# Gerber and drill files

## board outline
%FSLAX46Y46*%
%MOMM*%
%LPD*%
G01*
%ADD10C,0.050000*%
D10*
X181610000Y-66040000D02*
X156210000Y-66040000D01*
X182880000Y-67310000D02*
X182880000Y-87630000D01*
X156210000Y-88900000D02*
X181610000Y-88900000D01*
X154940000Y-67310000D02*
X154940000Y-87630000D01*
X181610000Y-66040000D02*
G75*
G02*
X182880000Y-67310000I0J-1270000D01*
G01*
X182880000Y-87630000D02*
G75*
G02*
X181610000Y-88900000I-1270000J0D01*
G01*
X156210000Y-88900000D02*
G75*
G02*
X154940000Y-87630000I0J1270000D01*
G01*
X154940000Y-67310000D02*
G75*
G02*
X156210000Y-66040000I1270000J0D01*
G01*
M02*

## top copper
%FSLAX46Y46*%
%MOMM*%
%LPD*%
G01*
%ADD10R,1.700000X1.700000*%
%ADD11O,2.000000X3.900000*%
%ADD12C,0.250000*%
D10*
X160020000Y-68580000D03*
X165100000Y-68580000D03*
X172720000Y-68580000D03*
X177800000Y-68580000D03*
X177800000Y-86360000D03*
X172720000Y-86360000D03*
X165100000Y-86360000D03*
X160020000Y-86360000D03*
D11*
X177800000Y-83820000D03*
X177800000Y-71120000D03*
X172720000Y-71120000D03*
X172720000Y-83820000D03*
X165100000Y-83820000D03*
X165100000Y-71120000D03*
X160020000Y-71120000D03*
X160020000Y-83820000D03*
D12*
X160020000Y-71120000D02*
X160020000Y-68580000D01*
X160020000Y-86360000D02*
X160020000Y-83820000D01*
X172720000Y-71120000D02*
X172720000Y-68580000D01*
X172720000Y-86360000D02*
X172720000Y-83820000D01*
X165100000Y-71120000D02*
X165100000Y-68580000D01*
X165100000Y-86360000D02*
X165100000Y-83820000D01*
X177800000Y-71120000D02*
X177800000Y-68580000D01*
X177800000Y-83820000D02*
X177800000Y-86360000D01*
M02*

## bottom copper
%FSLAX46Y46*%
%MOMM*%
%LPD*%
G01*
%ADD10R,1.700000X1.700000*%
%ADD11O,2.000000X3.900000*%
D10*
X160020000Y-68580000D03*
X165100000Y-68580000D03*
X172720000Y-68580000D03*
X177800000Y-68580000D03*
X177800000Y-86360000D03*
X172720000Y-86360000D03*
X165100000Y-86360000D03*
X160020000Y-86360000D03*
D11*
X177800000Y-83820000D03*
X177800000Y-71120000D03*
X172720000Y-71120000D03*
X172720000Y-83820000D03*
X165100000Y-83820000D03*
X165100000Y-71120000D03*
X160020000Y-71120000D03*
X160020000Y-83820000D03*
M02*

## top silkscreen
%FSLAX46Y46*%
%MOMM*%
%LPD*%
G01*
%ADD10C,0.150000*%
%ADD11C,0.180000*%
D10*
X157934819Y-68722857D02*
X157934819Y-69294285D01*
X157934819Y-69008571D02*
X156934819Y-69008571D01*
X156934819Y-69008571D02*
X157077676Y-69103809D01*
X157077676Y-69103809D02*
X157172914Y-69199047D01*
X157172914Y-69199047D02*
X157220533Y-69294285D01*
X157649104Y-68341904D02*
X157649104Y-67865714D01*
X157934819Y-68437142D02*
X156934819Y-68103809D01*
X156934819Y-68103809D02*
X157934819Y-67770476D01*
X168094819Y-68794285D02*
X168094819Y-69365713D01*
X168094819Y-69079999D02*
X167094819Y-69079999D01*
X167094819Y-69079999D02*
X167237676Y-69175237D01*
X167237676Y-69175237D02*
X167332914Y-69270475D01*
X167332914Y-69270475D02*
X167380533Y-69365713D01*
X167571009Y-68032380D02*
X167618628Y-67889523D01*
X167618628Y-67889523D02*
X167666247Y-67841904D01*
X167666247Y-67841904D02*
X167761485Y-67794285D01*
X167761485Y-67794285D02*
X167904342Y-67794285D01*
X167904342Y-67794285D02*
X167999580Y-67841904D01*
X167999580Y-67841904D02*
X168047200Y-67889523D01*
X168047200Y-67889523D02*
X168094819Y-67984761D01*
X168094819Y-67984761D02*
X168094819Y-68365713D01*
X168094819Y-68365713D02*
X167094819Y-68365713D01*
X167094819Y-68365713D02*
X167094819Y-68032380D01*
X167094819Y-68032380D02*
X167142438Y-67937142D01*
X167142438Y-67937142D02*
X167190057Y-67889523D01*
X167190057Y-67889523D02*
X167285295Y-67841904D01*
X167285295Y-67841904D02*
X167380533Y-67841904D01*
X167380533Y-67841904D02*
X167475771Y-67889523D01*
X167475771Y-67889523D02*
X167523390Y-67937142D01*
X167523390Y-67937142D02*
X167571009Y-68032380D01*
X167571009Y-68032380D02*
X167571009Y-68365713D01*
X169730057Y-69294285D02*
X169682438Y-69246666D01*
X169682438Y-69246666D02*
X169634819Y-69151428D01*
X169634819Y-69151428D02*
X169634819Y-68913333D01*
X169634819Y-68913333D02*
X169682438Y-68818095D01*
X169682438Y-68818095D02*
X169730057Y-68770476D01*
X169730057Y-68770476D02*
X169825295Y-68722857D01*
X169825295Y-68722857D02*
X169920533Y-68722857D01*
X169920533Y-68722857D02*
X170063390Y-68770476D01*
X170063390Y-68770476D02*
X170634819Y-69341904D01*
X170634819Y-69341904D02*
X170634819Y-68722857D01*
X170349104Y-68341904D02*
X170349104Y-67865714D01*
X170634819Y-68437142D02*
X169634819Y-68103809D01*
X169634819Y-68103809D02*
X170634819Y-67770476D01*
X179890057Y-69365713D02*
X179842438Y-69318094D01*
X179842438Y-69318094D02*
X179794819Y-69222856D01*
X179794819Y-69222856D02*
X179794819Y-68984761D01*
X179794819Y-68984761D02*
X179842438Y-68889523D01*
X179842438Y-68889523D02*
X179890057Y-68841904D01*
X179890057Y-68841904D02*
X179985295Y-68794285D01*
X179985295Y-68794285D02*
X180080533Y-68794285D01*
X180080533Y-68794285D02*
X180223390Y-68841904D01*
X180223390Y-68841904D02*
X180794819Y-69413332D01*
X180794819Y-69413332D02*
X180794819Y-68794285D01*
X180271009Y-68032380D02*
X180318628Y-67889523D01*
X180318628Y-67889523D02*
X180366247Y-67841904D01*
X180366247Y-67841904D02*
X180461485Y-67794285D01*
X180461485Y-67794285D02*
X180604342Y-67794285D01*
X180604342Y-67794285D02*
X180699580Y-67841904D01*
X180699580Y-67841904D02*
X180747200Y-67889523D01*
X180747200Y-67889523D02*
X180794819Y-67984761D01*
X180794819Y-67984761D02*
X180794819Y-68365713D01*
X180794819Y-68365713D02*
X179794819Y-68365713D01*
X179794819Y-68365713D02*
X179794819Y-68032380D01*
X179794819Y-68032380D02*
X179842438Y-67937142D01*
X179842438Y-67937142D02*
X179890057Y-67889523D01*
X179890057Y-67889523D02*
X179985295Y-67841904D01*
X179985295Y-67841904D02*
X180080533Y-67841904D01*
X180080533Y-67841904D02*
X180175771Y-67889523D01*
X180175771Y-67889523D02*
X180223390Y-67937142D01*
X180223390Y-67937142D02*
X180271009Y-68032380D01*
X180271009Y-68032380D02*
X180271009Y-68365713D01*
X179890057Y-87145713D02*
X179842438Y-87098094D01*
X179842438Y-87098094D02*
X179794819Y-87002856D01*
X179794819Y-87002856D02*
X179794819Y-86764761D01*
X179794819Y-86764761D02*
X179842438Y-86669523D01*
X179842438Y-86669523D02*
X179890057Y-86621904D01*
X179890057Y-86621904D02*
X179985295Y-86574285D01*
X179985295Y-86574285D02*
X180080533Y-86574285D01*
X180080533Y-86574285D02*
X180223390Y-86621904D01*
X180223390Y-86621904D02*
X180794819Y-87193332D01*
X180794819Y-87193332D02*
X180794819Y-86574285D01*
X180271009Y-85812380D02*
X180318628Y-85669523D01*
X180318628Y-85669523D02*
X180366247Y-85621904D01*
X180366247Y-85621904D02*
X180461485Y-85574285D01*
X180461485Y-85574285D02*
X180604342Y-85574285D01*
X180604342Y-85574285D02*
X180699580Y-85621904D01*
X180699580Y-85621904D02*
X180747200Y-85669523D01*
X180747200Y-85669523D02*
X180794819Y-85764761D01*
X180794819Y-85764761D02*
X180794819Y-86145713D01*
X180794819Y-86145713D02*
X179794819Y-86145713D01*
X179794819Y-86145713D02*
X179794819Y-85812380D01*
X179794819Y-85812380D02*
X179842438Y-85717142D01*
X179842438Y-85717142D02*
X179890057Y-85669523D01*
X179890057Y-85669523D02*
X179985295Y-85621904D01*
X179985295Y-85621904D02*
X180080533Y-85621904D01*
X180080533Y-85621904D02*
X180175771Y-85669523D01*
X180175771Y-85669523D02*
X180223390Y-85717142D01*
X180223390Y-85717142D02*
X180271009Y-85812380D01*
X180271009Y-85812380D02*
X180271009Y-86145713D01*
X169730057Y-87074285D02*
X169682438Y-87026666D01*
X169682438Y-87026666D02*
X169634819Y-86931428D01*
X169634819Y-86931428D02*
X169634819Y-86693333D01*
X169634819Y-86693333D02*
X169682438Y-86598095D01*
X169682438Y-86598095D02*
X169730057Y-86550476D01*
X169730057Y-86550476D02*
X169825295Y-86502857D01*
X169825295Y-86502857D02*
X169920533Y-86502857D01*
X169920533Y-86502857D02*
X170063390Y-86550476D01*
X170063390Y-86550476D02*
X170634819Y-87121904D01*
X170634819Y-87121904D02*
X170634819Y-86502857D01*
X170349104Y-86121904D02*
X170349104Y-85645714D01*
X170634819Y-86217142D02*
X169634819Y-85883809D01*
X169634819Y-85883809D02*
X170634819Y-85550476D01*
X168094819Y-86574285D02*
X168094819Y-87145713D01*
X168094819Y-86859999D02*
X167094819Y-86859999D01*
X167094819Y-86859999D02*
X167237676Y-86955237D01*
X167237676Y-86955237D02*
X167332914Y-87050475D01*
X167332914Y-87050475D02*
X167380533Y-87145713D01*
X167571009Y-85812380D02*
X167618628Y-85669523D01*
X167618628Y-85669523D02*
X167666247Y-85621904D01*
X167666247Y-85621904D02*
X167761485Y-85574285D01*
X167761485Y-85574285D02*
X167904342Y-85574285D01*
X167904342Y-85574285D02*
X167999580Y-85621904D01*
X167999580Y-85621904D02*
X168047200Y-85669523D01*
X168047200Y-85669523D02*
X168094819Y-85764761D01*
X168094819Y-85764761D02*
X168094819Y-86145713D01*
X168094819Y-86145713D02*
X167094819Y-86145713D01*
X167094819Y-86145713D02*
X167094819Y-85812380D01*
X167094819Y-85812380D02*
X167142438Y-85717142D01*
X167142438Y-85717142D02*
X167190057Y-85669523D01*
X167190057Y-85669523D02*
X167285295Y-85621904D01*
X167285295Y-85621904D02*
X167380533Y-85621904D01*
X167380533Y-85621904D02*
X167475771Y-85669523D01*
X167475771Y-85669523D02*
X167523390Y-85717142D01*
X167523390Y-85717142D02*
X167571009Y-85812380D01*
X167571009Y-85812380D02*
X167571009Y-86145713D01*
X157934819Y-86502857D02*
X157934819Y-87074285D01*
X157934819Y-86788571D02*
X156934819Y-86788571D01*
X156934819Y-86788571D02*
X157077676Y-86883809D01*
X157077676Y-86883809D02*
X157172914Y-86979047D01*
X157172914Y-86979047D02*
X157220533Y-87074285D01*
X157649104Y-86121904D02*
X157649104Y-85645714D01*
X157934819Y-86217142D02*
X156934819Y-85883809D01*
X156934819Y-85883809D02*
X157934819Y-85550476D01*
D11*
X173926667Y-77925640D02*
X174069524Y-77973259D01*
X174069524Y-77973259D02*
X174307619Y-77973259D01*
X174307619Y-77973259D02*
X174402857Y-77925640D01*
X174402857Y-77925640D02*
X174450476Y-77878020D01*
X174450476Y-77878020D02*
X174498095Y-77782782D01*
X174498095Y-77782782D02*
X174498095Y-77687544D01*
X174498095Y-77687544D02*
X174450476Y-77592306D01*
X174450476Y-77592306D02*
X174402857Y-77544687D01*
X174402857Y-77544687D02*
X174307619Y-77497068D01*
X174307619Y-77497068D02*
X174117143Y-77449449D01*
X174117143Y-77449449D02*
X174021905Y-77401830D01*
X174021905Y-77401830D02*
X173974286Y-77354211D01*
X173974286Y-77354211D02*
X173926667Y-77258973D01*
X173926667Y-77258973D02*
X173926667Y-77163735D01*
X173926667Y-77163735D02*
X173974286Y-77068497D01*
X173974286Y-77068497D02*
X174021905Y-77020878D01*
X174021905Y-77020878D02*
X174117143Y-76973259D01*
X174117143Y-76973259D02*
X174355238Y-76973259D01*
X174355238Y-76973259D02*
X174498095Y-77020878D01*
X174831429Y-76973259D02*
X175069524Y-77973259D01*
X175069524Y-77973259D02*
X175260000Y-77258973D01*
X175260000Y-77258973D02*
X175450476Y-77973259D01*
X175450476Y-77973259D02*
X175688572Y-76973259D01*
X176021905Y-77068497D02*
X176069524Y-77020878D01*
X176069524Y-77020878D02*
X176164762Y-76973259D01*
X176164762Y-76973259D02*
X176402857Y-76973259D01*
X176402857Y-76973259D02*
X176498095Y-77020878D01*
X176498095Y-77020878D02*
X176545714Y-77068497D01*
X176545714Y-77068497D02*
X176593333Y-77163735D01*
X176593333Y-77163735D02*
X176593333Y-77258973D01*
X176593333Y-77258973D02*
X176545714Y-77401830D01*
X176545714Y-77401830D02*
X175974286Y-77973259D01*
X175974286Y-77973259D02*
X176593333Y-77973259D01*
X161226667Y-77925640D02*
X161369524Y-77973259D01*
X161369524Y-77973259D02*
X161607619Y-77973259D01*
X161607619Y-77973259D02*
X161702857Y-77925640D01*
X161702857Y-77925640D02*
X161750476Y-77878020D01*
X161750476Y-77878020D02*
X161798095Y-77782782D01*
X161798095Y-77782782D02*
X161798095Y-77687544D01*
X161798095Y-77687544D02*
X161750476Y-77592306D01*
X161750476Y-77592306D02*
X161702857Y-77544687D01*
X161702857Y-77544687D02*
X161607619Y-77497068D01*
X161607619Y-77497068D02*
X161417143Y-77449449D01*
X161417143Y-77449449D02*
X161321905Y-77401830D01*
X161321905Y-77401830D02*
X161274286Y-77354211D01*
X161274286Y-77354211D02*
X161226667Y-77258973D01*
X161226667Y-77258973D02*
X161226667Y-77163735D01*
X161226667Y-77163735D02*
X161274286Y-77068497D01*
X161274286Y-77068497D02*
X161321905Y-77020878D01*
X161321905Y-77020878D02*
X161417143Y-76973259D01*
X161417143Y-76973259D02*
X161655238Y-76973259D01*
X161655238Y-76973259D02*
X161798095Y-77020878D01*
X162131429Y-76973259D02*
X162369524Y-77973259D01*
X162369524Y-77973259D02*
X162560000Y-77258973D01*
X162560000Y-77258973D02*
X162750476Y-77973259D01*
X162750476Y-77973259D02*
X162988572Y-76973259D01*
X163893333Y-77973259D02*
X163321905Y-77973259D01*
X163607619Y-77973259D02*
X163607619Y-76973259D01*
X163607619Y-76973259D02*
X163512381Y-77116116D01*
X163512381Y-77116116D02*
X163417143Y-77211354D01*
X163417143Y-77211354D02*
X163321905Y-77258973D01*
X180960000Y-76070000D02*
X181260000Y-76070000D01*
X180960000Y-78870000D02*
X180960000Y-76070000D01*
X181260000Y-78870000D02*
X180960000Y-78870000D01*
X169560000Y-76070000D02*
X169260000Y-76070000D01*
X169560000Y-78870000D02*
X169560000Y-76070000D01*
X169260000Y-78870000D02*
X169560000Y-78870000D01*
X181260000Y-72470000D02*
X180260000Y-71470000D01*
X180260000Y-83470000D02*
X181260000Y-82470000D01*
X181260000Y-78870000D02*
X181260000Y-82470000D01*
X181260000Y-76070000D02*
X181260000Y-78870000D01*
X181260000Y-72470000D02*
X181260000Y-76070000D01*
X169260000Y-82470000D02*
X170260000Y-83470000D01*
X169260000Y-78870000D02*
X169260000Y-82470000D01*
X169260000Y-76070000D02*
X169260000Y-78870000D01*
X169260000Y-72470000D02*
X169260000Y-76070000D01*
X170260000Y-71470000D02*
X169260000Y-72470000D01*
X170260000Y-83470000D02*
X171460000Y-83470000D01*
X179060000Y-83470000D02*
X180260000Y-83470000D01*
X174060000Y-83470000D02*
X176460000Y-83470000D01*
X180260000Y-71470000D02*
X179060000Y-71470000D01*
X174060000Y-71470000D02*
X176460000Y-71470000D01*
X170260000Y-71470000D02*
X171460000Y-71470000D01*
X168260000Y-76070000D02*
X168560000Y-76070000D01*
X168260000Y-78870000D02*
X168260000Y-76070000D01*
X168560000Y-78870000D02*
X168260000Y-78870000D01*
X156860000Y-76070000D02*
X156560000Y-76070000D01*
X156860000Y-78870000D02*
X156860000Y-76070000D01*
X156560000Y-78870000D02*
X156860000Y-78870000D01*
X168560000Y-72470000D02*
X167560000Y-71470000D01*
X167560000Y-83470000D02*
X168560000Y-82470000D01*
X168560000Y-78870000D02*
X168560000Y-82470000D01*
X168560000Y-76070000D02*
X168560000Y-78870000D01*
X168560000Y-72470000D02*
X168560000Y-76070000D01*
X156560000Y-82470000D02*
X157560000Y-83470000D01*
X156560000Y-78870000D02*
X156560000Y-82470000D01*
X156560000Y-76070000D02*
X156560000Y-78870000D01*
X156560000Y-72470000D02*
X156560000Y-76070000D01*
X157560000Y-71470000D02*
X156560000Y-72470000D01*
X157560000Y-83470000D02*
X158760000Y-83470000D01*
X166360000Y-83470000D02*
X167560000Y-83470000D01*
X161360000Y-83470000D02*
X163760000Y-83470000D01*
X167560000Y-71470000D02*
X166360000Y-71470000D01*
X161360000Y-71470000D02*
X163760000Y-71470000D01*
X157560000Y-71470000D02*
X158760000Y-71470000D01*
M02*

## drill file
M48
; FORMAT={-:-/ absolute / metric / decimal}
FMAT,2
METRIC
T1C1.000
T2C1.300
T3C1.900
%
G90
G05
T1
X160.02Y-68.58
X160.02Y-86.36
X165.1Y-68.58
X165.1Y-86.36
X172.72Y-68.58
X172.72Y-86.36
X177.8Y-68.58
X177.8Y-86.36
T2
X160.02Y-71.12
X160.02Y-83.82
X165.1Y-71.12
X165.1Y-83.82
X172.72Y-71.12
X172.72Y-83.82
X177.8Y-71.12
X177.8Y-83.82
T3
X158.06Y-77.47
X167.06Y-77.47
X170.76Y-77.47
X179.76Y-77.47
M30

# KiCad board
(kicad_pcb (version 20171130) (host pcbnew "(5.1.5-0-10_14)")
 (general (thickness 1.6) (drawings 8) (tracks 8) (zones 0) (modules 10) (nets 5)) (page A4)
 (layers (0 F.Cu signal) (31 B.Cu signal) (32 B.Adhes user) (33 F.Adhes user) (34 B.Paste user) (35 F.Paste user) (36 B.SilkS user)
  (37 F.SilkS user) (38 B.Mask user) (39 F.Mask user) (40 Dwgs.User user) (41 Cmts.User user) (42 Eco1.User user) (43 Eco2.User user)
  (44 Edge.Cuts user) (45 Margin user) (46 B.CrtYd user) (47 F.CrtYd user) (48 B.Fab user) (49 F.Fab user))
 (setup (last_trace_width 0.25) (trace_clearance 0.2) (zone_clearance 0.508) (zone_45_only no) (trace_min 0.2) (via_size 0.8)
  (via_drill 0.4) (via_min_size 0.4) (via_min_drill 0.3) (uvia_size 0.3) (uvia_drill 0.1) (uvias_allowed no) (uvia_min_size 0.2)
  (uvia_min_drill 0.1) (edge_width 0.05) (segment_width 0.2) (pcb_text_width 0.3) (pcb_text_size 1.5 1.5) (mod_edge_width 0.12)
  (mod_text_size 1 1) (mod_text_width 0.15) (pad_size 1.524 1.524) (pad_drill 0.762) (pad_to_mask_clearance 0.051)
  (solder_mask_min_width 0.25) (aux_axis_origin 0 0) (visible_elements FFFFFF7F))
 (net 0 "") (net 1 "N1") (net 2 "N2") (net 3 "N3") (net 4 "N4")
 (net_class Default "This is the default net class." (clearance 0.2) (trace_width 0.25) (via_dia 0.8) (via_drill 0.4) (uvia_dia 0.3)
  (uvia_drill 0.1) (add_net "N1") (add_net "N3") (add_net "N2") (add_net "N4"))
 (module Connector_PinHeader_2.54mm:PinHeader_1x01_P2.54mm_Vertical (layer F.Cu) (at 160.02 68.58 90)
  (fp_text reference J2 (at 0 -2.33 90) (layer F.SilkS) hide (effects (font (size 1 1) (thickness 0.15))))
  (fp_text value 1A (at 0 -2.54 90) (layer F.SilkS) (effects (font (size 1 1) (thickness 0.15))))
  (pad 1 thru_hole rect (at 0 0 90) (size 1.7 1.7) (drill 1) (layers *.Cu *.Mask) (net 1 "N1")))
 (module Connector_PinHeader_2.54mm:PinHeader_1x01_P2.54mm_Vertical (layer F.Cu) (at 165.1 68.58)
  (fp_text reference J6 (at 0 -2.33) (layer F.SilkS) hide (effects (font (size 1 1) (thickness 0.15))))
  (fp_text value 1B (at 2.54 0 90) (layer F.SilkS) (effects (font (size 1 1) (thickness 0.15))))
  (pad 1 thru_hole rect (at 0 0) (size 1.7 1.7) (drill 1) (layers *.Cu *.Mask) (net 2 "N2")))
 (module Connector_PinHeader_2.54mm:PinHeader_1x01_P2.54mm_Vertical (layer F.Cu) (at 172.72 68.58 90)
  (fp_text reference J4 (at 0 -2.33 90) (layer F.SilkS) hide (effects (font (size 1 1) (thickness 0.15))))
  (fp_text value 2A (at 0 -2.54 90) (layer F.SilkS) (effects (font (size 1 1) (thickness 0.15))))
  (pad 1 thru_hole rect (at 0 0 90) (size 1.7 1.7) (drill 1) (layers *.Cu *.Mask) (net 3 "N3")))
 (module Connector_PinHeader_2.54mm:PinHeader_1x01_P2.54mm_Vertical (layer F.Cu) (at 177.8 68.58)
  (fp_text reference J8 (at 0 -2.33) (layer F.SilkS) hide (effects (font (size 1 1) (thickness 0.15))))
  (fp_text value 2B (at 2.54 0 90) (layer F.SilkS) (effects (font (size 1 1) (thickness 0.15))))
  (pad 1 thru_hole rect (at 0 0) (size 1.7 1.7) (drill 1) (layers *.Cu *.Mask) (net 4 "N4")))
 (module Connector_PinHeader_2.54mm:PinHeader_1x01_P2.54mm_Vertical (layer F.Cu) (at 177.8 86.36)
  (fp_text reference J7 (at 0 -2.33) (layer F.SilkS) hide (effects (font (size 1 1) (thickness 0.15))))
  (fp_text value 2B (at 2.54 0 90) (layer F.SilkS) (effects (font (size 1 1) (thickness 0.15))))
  (pad 1 thru_hole rect (at 0 0) (size 1.7 1.7) (drill 1) (layers *.Cu *.Mask) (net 4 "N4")))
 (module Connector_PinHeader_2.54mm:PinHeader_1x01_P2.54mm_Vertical (layer F.Cu) (at 172.72 86.36 90)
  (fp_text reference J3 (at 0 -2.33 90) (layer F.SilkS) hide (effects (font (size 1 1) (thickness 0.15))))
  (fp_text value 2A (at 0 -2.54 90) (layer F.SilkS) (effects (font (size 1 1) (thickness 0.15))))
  (pad 1 thru_hole rect (at 0 0 90) (size 1.7 1.7) (drill 1) (layers *.Cu *.Mask) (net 3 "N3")))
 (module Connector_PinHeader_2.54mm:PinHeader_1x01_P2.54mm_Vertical (layer F.Cu) (at 165.1 86.36)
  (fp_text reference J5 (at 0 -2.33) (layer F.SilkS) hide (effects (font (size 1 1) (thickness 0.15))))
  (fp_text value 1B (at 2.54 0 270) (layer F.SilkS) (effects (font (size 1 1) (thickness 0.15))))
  (pad 1 thru_hole rect (at 0 0) (size 1.7 1.7) (drill 1) (layers *.Cu *.Mask) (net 2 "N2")))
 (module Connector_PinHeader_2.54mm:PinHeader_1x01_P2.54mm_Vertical (layer F.Cu) (at 160.02 86.36 90)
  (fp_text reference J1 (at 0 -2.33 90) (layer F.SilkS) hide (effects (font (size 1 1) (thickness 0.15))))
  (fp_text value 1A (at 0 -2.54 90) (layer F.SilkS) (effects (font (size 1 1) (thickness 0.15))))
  (pad 1 thru_hole rect (at 0 0 90) (size 1.7 1.7) (drill 1) (layers *.Cu *.Mask) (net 1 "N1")))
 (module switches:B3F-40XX (layer F.Cu) (at 175.26 77.47 90)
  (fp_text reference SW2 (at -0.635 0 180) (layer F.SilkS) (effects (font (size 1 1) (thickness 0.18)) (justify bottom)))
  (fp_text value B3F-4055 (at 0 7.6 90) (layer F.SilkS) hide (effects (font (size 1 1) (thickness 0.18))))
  (fp_line (start 1.4 5.7) (end 1.4 6) (layer F.SilkS) (width 0.18))
  (fp_line (start -1.4 5.7) (end 1.4 5.7) (layer F.SilkS) (width 0.18))
  (fp_line (start -1.4 6) (end -1.4 5.7) (layer F.SilkS) (width 0.18))
  (fp_line (start 1.4 -5.7) (end 1.4 -6) (layer F.SilkS) (width 0.18))
  (fp_line (start -1.4 -5.7) (end 1.4 -5.7) (layer F.SilkS) (width 0.18))
  (fp_line (start -1.4 -6) (end -1.4 -5.7) (layer F.SilkS) (width 0.18)) (fp_line (start 5 6) (end 6 5) (layer F.SilkS) (width 0.18))
  (fp_line (start -6 5) (end -5 6) (layer F.SilkS) (width 0.18))
  (fp_line (start -1.4 6) (end -5 6) (layer F.SilkS) (width 0.18))
  (fp_line (start 1.4 6) (end -1.4 6) (layer F.SilkS) (width 0.18))
  (fp_line (start 5 6) (end 1.4 6) (layer F.SilkS) (width 0.18))
  (fp_line (start -5 -6) (end -6 -5) (layer F.SilkS) (width 0.18))
  (fp_line (start -1.4 -6) (end -5 -6) (layer F.SilkS) (width 0.18))
  (fp_line (start 1.4 -6) (end -1.4 -6) (layer F.SilkS) (width 0.18))
  (fp_line (start 5 -6) (end 1.4 -6) (layer F.SilkS) (width 0.18))
  (fp_line (start 6 -5) (end 5 -6) (layer F.SilkS) (width 0.18))
  (fp_line (start -6 -5) (end -6 -3.8) (layer F.SilkS) (width 0.18))
  (fp_line (start -6 3.8) (end -6 5) (layer F.SilkS) (width 0.18))
  (fp_line (start -6 -1.2) (end -6 1.2) (layer F.SilkS) (width 0.18))
  (fp_line (start 6 5) (end 6 3.8) (layer F.SilkS) (width 0.18))
  (fp_line (start 6 -1.2) (end 6 1.2) (layer F.SilkS) (width 0.18))
  (fp_line (start 6 -5) (end 6 -3.8) (layer F.SilkS) (width 0.18))
  (pad "" np_thru_hole circle (at 0 -4.5 90) (size 1.9 1.9) (drill 1.9) (layers *.Cu))
  (pad "" np_thru_hole circle (at 0 4.5 90) (size 1.9 1.9) (drill 1.9) (layers *.Cu))
  (pad 2 thru_hole oval (at -6.35 2.54 90) (size 3.9 2) (drill 1.3) (layers *.Cu *.Mask) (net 4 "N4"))
  (pad 2 thru_hole oval (at 6.35 2.54 90) (size 3.9 2) (drill 1.3) (layers *.Cu *.Mask) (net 4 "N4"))
  (pad 1 thru_hole oval (at 6.35 -2.54 90) (size 3.9 2) (drill 1.3) (layers *.Cu *.Mask) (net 3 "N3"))
  (pad 1 thru_hole oval (at -6.35 -2.54 90) (size 3.9 2) (drill 1.3) (layers *.Cu *.Mask) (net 3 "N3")))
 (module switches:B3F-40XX (layer F.Cu) (at 162.56 77.47 90)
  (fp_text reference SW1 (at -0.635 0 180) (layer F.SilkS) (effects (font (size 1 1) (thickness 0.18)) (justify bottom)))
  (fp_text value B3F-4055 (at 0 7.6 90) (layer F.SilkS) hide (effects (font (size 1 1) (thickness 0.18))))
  (fp_line (start 1.4 5.7) (end 1.4 6) (layer F.SilkS) (width 0.18))
  (fp_line (start -1.4 5.7) (end 1.4 5.7) (layer F.SilkS) (width 0.18))
  (fp_line (start -1.4 6) (end -1.4 5.7) (layer F.SilkS) (width 0.18))
  (fp_line (start 1.4 -5.7) (end 1.4 -6) (layer F.SilkS) (width 0.18))
  (fp_line (start -1.4 -5.7) (end 1.4 -5.7) (layer F.SilkS) (width 0.18))
  (fp_line (start -1.4 -6) (end -1.4 -5.7) (layer F.SilkS) (width 0.18)) (fp_line (start 5 6) (end 6 5) (layer F.SilkS) (width 0.18))
  (fp_line (start -6 5) (end -5 6) (layer F.SilkS) (width 0.18))
  (fp_line (start -1.4 6) (end -5 6) (layer F.SilkS) (width 0.18))
  (fp_line (start 1.4 6) (end -1.4 6) (layer F.SilkS) (width 0.18))
  (fp_line (start 5 6) (end 1.4 6) (layer F.SilkS) (width 0.18))
  (fp_line (start -5 -6) (end -6 -5) (layer F.SilkS) (width 0.18))
  (fp_line (start -1.4 -6) (end -5 -6) (layer F.SilkS) (width 0.18))
  (fp_line (start 1.4 -6) (end -1.4 -6) (layer F.SilkS) (width 0.18))
  (fp_line (start 5 -6) (end 1.4 -6) (layer F.SilkS) (width 0.18))
  (fp_line (start 6 -5) (end 5 -6) (layer F.SilkS) (width 0.18))
  (fp_line (start -6 -5) (end -6 -3.8) (layer F.SilkS) (width 0.18))
  (fp_line (start -6 3.8) (end -6 5) (layer F.SilkS) (width 0.18))
  (fp_line (start -6 -1.2) (end -6 1.2) (layer F.SilkS) (width 0.18))
  (fp_line (start 6 5) (end 6 3.8) (layer F.SilkS) (width 0.18))
  (fp_line (start 6 -1.2) (end 6 1.2) (layer F.SilkS) (width 0.18))
  (fp_line (start 6 -5) (end 6 -3.8) (layer F.SilkS) (width 0.18))
  (pad "" np_thru_hole circle (at 0 -4.5 90) (size 1.9 1.9) (drill 1.9) (layers *.Cu))
  (pad "" np_thru_hole circle (at 0 4.5 90) (size 1.9 1.9) (drill 1.9) (layers *.Cu))
  (pad 2 thru_hole oval (at -6.35 2.54 90) (size 3.9 2) (drill 1.3) (layers *.Cu *.Mask) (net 2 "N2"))
  (pad 2 thru_hole oval (at 6.35 2.54 90) (size 3.9 2) (drill 1.3) (layers *.Cu *.Mask) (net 2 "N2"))
  (pad 1 thru_hole oval (at 6.35 -2.54 90) (size 3.9 2) (drill 1.3) (layers *.Cu *.Mask) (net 1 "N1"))
  (pad 1 thru_hole oval (at -6.35 -2.54 90) (size 3.9 2) (drill 1.3) (layers *.Cu *.Mask) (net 1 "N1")))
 (gr_line (start 181.61 66.04) (end 156.21 66.04) (layer Edge.Cuts) (width 0.05))
 (gr_line (start 182.88 67.31) (end 182.88 87.63) (layer Edge.Cuts) (width 0.05))
 (gr_line (start 156.21 88.9) (end 181.61 88.9) (layer Edge.Cuts) (width 0.05))
 (gr_line (start 154.94 67.31) (end 154.94 87.63) (layer Edge.Cuts) (width 0.05))
 (gr_arc (start 181.61 67.31) (end 182.88 67.31) (angle -90) (layer Edge.Cuts) (width 0.05))
 (gr_arc (start 181.61 87.63) (end 181.61 88.9) (angle -90) (layer Edge.Cuts) (width 0.05))
 (gr_arc (start 156.21 87.63) (end 154.94 87.63) (angle -90) (layer Edge.Cuts) (width 0.05))
 (gr_arc (start 156.21 67.31) (end 156.21 66.04) (angle -90) (layer Edge.Cuts) (width 0.05))
 (segment (start 160.02 71.12) (end 160.02 68.58) (width 0.25) (layer F.Cu) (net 1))
 (segment (start 160.02 86.36) (end 160.02 83.82) (width 0.25) (layer F.Cu) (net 1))
 (segment (start 172.72 71.12) (end 172.72 68.58) (width 0.25) (layer F.Cu) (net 3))
 (segment (start 172.72 86.36) (end 172.72 83.82) (width 0.25) (layer F.Cu) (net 3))
 (segment (start 165.1 71.12) (end 165.1 68.58) (width 0.25) (layer F.Cu) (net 2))
 (segment (start 165.1 86.36) (end 165.1 83.82) (width 0.25) (layer F.Cu) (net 2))
 (segment (start 177.8 71.12) (end 177.8 68.58) (width 0.25) (layer F.Cu) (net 4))
 (segment (start 177.8 83.82) (end 177.8 86.36) (width 0.25) (layer F.Cu) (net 4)))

